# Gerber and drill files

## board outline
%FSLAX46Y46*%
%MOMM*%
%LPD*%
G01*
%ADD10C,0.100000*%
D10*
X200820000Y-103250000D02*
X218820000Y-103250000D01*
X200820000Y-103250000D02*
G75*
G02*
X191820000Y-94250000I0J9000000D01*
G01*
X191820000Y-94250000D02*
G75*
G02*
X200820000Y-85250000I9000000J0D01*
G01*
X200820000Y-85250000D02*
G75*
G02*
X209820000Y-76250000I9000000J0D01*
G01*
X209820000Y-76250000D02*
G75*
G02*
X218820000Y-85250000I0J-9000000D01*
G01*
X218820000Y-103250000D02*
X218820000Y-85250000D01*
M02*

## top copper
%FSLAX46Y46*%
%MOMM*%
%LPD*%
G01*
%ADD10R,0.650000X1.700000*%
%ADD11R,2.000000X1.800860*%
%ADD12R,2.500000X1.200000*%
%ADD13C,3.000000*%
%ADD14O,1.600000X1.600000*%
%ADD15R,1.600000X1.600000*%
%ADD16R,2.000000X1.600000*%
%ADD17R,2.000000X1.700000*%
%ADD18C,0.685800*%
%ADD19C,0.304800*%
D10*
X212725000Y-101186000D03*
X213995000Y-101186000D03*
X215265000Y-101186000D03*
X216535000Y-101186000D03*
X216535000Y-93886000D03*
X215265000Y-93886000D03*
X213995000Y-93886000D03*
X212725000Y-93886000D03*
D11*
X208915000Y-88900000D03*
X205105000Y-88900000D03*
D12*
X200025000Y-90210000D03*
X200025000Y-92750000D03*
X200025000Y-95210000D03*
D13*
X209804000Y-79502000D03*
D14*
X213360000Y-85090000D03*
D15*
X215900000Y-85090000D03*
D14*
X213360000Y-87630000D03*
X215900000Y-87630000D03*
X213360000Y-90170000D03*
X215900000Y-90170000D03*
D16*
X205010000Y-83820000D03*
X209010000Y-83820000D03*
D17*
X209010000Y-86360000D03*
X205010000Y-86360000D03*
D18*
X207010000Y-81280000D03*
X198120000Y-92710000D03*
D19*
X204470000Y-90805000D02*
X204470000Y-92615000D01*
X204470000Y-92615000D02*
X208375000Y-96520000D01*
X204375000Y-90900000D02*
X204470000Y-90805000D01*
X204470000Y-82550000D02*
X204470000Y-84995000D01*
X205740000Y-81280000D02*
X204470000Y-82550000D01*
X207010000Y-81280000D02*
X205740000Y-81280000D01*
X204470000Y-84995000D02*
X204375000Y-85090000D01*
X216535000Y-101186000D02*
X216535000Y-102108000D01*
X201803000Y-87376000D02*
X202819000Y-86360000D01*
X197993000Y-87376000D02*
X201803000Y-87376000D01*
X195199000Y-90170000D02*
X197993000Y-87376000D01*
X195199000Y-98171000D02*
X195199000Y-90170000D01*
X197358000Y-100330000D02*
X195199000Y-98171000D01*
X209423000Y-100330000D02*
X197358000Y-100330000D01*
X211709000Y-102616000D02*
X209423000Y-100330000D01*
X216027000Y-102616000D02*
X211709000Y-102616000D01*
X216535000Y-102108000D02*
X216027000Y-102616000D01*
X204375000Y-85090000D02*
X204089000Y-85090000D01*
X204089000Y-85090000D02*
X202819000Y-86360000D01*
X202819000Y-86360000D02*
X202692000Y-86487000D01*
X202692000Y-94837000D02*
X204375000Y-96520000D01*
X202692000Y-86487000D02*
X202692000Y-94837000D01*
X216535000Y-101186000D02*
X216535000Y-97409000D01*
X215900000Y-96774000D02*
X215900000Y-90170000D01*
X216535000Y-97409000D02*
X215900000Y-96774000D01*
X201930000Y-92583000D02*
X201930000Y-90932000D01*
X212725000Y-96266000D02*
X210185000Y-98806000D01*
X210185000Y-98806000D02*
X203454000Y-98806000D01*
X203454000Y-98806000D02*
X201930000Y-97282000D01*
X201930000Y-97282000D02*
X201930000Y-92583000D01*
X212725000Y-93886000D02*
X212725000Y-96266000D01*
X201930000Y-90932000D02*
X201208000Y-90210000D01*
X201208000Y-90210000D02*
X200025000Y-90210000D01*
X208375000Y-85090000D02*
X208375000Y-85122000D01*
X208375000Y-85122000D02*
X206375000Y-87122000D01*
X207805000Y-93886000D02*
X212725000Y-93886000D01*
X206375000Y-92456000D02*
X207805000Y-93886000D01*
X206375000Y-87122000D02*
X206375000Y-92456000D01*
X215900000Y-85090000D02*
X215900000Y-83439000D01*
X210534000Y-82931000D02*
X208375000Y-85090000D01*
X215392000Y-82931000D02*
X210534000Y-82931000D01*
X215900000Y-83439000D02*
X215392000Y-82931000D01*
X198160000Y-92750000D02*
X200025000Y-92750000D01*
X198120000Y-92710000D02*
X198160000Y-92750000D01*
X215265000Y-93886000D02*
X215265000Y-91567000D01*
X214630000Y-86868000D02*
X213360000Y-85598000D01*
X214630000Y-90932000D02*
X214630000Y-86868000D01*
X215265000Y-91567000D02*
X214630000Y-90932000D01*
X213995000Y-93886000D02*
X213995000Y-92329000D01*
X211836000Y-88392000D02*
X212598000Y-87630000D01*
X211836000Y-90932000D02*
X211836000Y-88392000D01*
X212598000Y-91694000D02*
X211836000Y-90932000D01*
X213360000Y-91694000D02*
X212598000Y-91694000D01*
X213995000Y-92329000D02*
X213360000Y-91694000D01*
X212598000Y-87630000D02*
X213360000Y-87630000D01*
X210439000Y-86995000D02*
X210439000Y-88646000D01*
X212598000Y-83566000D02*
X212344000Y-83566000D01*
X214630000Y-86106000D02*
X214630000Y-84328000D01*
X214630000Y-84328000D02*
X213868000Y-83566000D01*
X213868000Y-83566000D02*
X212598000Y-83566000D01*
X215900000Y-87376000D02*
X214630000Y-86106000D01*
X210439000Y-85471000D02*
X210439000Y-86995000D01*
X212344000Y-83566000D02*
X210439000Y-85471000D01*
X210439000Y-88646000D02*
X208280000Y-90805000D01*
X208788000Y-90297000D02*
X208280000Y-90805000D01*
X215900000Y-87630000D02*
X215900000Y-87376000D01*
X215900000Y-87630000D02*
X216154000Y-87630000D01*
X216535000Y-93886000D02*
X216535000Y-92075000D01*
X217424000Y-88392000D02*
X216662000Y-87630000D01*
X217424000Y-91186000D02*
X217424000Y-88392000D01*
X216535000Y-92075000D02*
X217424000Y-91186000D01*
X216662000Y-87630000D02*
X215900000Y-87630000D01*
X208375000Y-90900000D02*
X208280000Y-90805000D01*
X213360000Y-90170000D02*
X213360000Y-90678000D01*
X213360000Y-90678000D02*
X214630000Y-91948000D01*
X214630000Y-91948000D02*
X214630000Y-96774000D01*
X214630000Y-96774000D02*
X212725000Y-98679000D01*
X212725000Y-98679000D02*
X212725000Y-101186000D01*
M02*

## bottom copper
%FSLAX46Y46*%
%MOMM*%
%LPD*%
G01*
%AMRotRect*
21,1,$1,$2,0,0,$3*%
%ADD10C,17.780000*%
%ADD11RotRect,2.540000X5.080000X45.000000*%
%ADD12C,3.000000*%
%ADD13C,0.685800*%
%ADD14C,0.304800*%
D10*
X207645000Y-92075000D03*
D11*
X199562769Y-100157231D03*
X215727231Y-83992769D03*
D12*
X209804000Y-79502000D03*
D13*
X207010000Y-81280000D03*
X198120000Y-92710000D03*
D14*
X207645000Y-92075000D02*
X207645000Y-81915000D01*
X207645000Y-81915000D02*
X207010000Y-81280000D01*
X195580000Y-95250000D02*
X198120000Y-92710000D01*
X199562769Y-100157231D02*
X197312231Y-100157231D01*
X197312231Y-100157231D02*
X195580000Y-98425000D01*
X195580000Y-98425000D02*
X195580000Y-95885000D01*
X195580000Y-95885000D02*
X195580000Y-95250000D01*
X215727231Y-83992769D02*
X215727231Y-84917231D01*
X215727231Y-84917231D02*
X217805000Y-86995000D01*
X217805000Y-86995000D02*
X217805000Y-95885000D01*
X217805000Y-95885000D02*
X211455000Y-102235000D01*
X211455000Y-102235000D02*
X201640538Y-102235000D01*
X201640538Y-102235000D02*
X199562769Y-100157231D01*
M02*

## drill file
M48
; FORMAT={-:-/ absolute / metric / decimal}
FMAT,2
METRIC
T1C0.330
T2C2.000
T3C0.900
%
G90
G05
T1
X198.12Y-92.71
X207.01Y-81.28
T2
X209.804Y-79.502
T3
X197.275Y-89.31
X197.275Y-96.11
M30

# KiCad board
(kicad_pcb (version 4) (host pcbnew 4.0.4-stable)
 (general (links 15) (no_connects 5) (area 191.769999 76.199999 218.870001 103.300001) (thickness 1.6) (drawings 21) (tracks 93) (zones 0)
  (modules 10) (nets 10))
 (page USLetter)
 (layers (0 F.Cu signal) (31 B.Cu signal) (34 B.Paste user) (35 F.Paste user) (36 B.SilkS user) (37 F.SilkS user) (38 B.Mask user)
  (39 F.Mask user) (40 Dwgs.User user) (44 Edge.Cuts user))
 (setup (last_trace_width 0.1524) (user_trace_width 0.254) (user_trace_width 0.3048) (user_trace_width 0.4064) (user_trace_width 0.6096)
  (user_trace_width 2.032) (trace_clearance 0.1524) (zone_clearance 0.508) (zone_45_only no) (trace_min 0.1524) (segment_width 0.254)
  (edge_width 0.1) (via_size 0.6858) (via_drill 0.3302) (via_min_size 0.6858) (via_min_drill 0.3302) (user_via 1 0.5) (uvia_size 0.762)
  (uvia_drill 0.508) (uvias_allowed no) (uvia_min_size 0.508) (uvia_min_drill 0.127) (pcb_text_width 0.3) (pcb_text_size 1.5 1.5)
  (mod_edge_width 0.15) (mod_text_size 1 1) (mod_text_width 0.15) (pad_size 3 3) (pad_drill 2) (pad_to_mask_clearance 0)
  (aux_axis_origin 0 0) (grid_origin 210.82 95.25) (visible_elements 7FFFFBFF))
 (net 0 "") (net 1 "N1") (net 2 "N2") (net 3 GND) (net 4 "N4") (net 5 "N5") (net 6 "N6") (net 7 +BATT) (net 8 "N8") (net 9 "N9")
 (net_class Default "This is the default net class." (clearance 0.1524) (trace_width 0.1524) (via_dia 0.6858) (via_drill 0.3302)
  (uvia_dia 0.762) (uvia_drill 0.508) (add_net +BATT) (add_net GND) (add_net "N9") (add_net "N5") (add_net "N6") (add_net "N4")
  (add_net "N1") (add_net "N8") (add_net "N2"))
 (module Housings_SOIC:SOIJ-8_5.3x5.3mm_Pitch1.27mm (layer F.Cu) (at 214.63 97.536 90)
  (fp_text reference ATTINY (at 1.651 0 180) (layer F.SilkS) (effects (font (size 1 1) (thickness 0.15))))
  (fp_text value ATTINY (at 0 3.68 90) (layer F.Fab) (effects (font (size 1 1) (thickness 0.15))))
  (pad 1 smd rect (at -3.65 -1.905 90) (size 1.7 0.65) (layers F.Cu F.Paste F.Mask) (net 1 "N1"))
  (pad 2 smd rect (at -3.65 -0.635 90) (size 1.7 0.65) (layers F.Cu F.Paste F.Mask) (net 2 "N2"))
  (pad 3 smd rect (at -3.65 0.635 90) (size 1.7 0.65) (layers F.Cu F.Paste F.Mask))
  (pad 4 smd rect (at -3.65 1.905 90) (size 1.7 0.65) (layers F.Cu F.Paste F.Mask) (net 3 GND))
  (pad 5 smd rect (at 3.65 1.905 90) (size 1.7 0.65) (layers F.Cu F.Paste F.Mask) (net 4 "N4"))
  (pad 6 smd rect (at 3.65 0.635 90) (size 1.7 0.65) (layers F.Cu F.Paste F.Mask) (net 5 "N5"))
  (pad 7 smd rect (at 3.65 -0.635 90) (size 1.7 0.65) (layers F.Cu F.Paste F.Mask) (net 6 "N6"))
  (pad 8 smd rect (at 3.65 -1.905 90) (size 1.7 0.65) (layers F.Cu F.Paste F.Mask) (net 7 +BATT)))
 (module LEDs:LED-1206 (layer F.Cu) (at 207.01 88.9)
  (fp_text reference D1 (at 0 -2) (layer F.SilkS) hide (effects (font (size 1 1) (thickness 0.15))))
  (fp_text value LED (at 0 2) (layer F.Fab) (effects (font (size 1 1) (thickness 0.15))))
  (pad 2 smd rect (at 1.905 0 180) (size 2 1.80086) (layers F.Cu F.Paste F.Mask) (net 4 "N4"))
  (pad 1 smd rect (at -1.905 0 180) (size 2 1.80086) (layers F.Cu F.Paste F.Mask) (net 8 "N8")))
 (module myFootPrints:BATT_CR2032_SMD (layer B.Cu) (at 207.645 92.075 45)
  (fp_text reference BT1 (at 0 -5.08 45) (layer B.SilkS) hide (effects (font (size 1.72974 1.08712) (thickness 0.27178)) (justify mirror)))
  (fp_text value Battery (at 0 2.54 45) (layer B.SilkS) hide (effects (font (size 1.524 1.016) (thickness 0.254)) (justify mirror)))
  (pad 2 smd circle (at 0 0 45) (size 17.78 17.78) (layers B.Cu B.Paste B.Mask) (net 3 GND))
  (pad 1 smd rect (at -11.43 0 45) (size 2.54 5.08) (layers B.Cu B.Paste B.Mask) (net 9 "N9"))
  (pad 1 smd rect (at 11.43 0 45) (size 2.54 5.08) (layers B.Cu B.Paste B.Mask) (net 9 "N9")))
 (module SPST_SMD (layer F.Cu) (at 200.025 92.71 270)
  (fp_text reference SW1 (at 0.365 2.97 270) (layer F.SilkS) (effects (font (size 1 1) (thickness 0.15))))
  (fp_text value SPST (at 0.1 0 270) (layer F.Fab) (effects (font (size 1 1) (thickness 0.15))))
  (pad "" np_thru_hole circle (at 3.4 2.75 270) (size 0.9 0.9) (drill 0.9) (layers *.Cu *.Mask))
  (pad 1 smd rect (at -2.5 0 270) (size 1.2 2.5) (layers F.Cu F.Paste F.Mask) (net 7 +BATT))
  (pad 2 smd rect (at 0.04 0 270) (size 1.2 2.5) (layers F.Cu F.Paste F.Mask) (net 9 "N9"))
  (pad 3 smd rect (at 2.5 0 270) (size 1.2 2.5) (layers F.Cu F.Paste F.Mask))
  (pad "" np_thru_hole circle (at -3.4 2.75 270) (size 0.9 0.9) (drill 0.9) (layers *.Cu *.Mask)))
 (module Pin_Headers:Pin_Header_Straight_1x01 (layer F.Cu) (at 209.804 79.502)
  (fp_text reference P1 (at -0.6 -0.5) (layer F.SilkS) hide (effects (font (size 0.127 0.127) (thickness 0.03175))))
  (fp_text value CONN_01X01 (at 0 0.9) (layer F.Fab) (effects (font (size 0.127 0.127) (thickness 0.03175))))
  (pad "" thru_hole circle (at 0 0) (size 3 3) (drill 2) (layers *.Cu *.Mask)))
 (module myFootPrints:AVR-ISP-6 (layer F.Cu) (at 213.36 85.09)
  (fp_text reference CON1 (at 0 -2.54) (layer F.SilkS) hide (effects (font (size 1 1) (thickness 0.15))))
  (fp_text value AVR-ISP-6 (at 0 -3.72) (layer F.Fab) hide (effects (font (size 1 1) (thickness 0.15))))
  (pad 1 smd oval (at 0 0) (size 1.6 1.6) (layers F.Cu F.Paste F.Mask) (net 5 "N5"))
  (pad 2 smd rect (at 2.54 0) (size 1.6 1.6) (layers F.Cu F.Paste F.Mask) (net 7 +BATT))
  (pad 3 smd oval (at 0 2.54) (size 1.6 1.6) (layers F.Cu F.Paste F.Mask) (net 6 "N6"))
  (pad 4 smd oval (at 2.54 2.54) (size 1.6 1.6) (layers F.Cu F.Paste F.Mask) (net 4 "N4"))
  (pad 5 smd oval (at 0 5.08) (size 1.6 1.6) (layers F.Cu F.Paste F.Mask) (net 1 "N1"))
  (pad 6 smd oval (at 2.54 5.08) (size 1.6 1.6) (layers F.Cu F.Paste F.Mask) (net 3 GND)))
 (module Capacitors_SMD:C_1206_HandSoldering (layer F.Cu) (at 207.01 83.82)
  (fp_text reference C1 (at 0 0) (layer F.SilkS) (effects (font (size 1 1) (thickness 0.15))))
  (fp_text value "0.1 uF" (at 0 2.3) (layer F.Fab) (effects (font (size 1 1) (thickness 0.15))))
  (pad 1 smd rect (at -2 0) (size 2 1.6) (layers F.Cu F.Paste F.Mask) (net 3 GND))
  (pad 2 smd rect (at 2 0) (size 2 1.6) (layers F.Cu F.Paste F.Mask) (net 7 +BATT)))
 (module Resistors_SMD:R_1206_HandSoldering (layer F.Cu) (at 207.01 86.36 180)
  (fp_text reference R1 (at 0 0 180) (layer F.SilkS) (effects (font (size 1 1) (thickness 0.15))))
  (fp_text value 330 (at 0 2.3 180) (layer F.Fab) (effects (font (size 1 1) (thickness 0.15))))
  (pad 1 smd rect (at -2 0 180) (size 2 1.7) (layers F.Cu F.Paste F.Mask) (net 8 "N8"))
  (pad 2 smd rect (at 2 0 180) (size 2 1.7) (layers F.Cu F.Paste F.Mask) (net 3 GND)))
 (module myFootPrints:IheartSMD (layer F.Cu) (at 242.82 83.25)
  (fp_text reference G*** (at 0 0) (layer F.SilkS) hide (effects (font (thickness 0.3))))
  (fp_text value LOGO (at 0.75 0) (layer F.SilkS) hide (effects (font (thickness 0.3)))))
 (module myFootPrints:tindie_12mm (layer F.Cu) (at 206.82 96.25)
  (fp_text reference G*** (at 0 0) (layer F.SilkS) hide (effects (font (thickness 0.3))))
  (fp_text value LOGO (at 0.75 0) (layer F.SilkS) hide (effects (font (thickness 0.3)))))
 (gr_line (start 200.82 103.25) (end 218.82 103.25) (angle 90) (layer Edge.Cuts) (width 0.1))
 (gr_arc (start 200.82 94.25) (end 200.82 103.25) (angle 90) (layer Edge.Cuts) (width 0.1))
 (gr_arc (start 200.82 94.25) (end 191.82 94.25) (angle 90) (layer Edge.Cuts) (width 0.1))
 (gr_arc (start 209.82 85.25) (end 200.82 85.25) (angle 90) (layer Edge.Cuts) (width 0.1))
 (gr_arc (start 209.82 85.25) (end 209.82 76.25) (angle 90) (layer Edge.Cuts) (width 0.1))
 (gr_line (start 218.82 103.25) (end 218.82 85.25) (angle 90) (layer Edge.Cuts) (width 0.1))
 (segment (start 204.47 90.805) (end 204.47 92.615) (width 0.3048) (layer F.Cu) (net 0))
 (segment (start 204.47 92.615) (end 208.375 96.52) (width 0.3048) (layer F.Cu) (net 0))
 (segment (start 204.375 90.9) (end 204.47 90.805) (width 0.3048) (layer F.Cu) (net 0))
 (segment (start 207.645 92.075) (end 207.645 81.915) (width 0.3048) (layer B.Cu) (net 3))
 (segment (start 204.47 82.55) (end 204.47 84.995) (width 0.3048) (layer F.Cu) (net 3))
 (segment (start 205.74 81.28) (end 204.47 82.55) (width 0.3048) (layer F.Cu) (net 3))
 (segment (start 207.01 81.28) (end 205.74 81.28) (width 0.3048) (layer F.Cu) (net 3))
 (via (at 207.01 81.28) (size 0.6858) (drill 0.3302) (layers F.Cu B.Cu) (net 3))
 (segment (start 207.645 81.915) (end 207.01 81.28) (width 0.3048) (layer B.Cu) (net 3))
 (segment (start 204.47 84.995) (end 204.375 85.09) (width 0.3048) (layer F.Cu) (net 3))
 (segment (start 216.535 101.186) (end 216.535 102.108) (width 0.3048) (layer F.Cu) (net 3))
 (segment (start 201.803 87.376) (end 202.819 86.36) (width 0.3048) (layer F.Cu) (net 3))
 (segment (start 197.993 87.376) (end 201.803 87.376) (width 0.3048) (layer F.Cu) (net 3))
 (segment (start 195.199 90.17) (end 197.993 87.376) (width 0.3048) (layer F.Cu) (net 3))
 (segment (start 195.199 98.171) (end 195.199 90.17) (width 0.3048) (layer F.Cu) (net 3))
 (segment (start 197.358 100.33) (end 195.199 98.171) (width 0.3048) (layer F.Cu) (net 3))
 (segment (start 209.423 100.33) (end 197.358 100.33) (width 0.3048) (layer F.Cu) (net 3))
 (segment (start 211.709 102.616) (end 209.423 100.33) (width 0.3048) (layer F.Cu) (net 3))
 (segment (start 216.027 102.616) (end 211.709 102.616) (width 0.3048) (layer F.Cu) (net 3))
 (segment (start 216.535 102.108) (end 216.027 102.616) (width 0.3048) (layer F.Cu) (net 3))
 (segment (start 204.375 85.09) (end 204.089 85.09) (width 0.3048) (layer F.Cu) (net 3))
 (segment (start 204.089 85.09) (end 202.819 86.36) (width 0.3048) (layer F.Cu) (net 3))
 (segment (start 202.819 86.36) (end 202.692 86.487) (width 0.3048) (layer F.Cu) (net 3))
 (segment (start 202.692 94.837) (end 204.375 96.52) (width 0.3048) (layer F.Cu) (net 3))
 (segment (start 202.692 86.487) (end 202.692 94.837) (width 0.3048) (layer F.Cu) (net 3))
 (segment (start 216.535 101.186) (end 216.535 97.409) (width 0.3048) (layer F.Cu) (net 3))
 (segment (start 215.9 96.774) (end 215.9 90.17) (width 0.3048) (layer F.Cu) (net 3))
 (segment (start 216.535 97.409) (end 215.9 96.774) (width 0.3048) (layer F.Cu) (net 3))
 (segment (start 201.93 92.583) (end 201.93 90.932) (width 0.3048) (layer F.Cu) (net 7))
 (segment (start 212.725 96.266) (end 210.185 98.806) (width 0.3048) (layer F.Cu) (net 7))
 (segment (start 210.185 98.806) (end 203.454 98.806) (width 0.3048) (layer F.Cu) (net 7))
 (segment (start 203.454 98.806) (end 201.93 97.282) (width 0.3048) (layer F.Cu) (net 7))
 (segment (start 201.93 97.282) (end 201.93 92.583) (width 0.3048) (layer F.Cu) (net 7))
 (segment (start 212.725 93.886) (end 212.725 96.266) (width 0.3048) (layer F.Cu) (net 7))
 (segment (start 201.93 90.932) (end 201.208 90.21) (width 0.3048) (layer F.Cu) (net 7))
 (segment (start 201.208 90.21) (end 200.025 90.21) (width 0.3048) (layer F.Cu) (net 7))
 (segment (start 208.375 85.09) (end 208.375 85.122) (width 0.3048) (layer F.Cu) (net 7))
 (segment (start 208.375 85.122) (end 206.375 87.122) (width 0.3048) (layer F.Cu) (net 7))
 (segment (start 207.805 93.886) (end 212.725 93.886) (width 0.3048) (layer F.Cu) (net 7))
 (segment (start 206.375 92.456) (end 207.805 93.886) (width 0.3048) (layer F.Cu) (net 7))
 (segment (start 206.375 87.122) (end 206.375 92.456) (width 0.3048) (layer F.Cu) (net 7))
 (segment (start 215.9 85.09) (end 215.9 83.439) (width 0.3048) (layer F.Cu) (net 7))
 (segment (start 210.534 82.931) (end 208.375 85.09) (width 0.3048) (layer F.Cu) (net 7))
 (segment (start 215.392 82.931) (end 210.534 82.931) (width 0.3048) (layer F.Cu) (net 7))
 (segment (start 215.9 83.439) (end 215.392 82.931) (width 0.3048) (layer F.Cu) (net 7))
 (segment (start 195.58 95.25) (end 198.12 92.71) (width 0.3048) (layer B.Cu) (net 9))
 (segment (start 198.16 92.75) (end 200.025 92.75) (width 0.3048) (layer F.Cu) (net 9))
 (via (at 198.12 92.71) (size 0.6858) (drill 0.3302) (layers F.Cu B.Cu) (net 9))
 (segment (start 198.12 92.71) (end 198.16 92.75) (width 0.3048) (layer F.Cu) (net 9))
 (segment (start 199.562769 100.157231) (end 197.312231 100.157231) (width 0.3048) (layer B.Cu) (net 9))
 (segment (start 197.312231 100.157231) (end 195.58 98.425) (width 0.3048) (layer B.Cu) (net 9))
 (segment (start 195.58 98.425) (end 195.58 95.885) (width 0.3048) (layer B.Cu) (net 9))
 (segment (start 195.58 95.885) (end 195.58 95.25) (width 0.3048) (layer B.Cu) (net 9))
 (segment (start 215.727231 83.992769) (end 215.727231 84.917231) (width 0.3048) (layer B.Cu) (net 9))
 (segment (start 215.727231 84.917231) (end 217.805 86.995) (width 0.3048) (layer B.Cu) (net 9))
 (segment (start 217.805 86.995) (end 217.805 95.885) (width 0.3048) (layer B.Cu) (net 9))
 (segment (start 217.805 95.885) (end 211.455 102.235) (width 0.3048) (layer B.Cu) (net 9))
 (segment (start 211.455 102.235) (end 201.640538 102.235) (width 0.3048) (layer B.Cu) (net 9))
 (segment (start 201.640538 102.235) (end 199.562769 100.157231) (width 0.3048) (layer B.Cu) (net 9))
 (segment (start 215.265 93.886) (end 215.265 91.567) (width 0.3048) (layer F.Cu) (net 5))
 (segment (start 214.63 86.868) (end 213.36 85.598) (width 0.3048) (layer F.Cu) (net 5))
 (segment (start 214.63 90.932) (end 214.63 86.868) (width 0.3048) (layer F.Cu) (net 5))
 (segment (start 215.265 91.567) (end 214.63 90.932) (width 0.3048) (layer F.Cu) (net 5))
 (segment (start 213.995 93.886) (end 213.995 92.329) (width 0.3048) (layer F.Cu) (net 6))
 (segment (start 211.836 88.392) (end 212.598 87.63) (width 0.3048) (layer F.Cu) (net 6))
 (segment (start 211.836 90.932) (end 211.836 88.392) (width 0.3048) (layer F.Cu) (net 6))
 (segment (start 212.598 91.694) (end 211.836 90.932) (width 0.3048) (layer F.Cu) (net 6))
 (segment (start 213.36 91.694) (end 212.598 91.694) (width 0.3048) (layer F.Cu) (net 6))
 (segment (start 213.995 92.329) (end 213.36 91.694) (width 0.3048) (layer F.Cu) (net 6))
 (segment (start 212.598 87.63) (end 213.36 87.63) (width 0.3048) (layer F.Cu) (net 6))
 (segment (start 210.439 86.995) (end 210.439 88.646) (width 0.3048) (layer F.Cu) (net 4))
 (segment (start 212.598 83.566) (end 212.344 83.566) (width 0.3048) (layer F.Cu) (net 4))
 (segment (start 214.63 86.106) (end 214.63 84.328) (width 0.3048) (layer F.Cu) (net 4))
 (segment (start 214.63 84.328) (end 213.868 83.566) (width 0.3048) (layer F.Cu) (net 4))
 (segment (start 213.868 83.566) (end 212.598 83.566) (width 0.3048) (layer F.Cu) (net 4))
 (segment (start 215.9 87.376) (end 214.63 86.106) (width 0.3048) (layer F.Cu) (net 4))
 (segment (start 210.439 85.471) (end 210.439 86.995) (width 0.3048) (layer F.Cu) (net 4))
 (segment (start 212.344 83.566) (end 210.439 85.471) (width 0.3048) (layer F.Cu) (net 4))
 (segment (start 210.439 88.646) (end 208.28 90.805) (width 0.3048) (layer F.Cu) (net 4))
 (segment (start 208.788 90.297) (end 208.28 90.805) (width 0.3048) (layer F.Cu) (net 4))
 (segment (start 215.9 87.63) (end 215.9 87.376) (width 0.3048) (layer F.Cu) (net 4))
 (segment (start 215.9 87.63) (end 216.154 87.63) (width 0.3048) (layer F.Cu) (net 4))
 (segment (start 216.535 93.886) (end 216.535 92.075) (width 0.3048) (layer F.Cu) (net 4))
 (segment (start 217.424 88.392) (end 216.662 87.63) (width 0.3048) (layer F.Cu) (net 4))
 (segment (start 217.424 91.186) (end 217.424 88.392) (width 0.3048) (layer F.Cu) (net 4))
 (segment (start 216.535 92.075) (end 217.424 91.186) (width 0.3048) (layer F.Cu) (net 4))
 (segment (start 216.662 87.63) (end 215.9 87.63) (width 0.3048) (layer F.Cu) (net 4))
 (segment (start 208.375 90.9) (end 208.28 90.805) (width 0.3048) (layer F.Cu) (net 4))
 (segment (start 213.36 90.17) (end 213.36 90.678) (width 0.3048) (layer F.Cu) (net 1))
 (segment (start 213.36 90.678) (end 214.63 91.948) (width 0.3048) (layer F.Cu) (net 1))
 (segment (start 214.63 91.948) (end 214.63 96.774) (width 0.3048) (layer F.Cu) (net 1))
 (segment (start 214.63 96.774) (end 212.725 98.679) (width 0.3048) (layer F.Cu) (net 1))
 (segment (start 212.725 98.679) (end 212.725 101.186) (width 0.3048) (layer F.Cu) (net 1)))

